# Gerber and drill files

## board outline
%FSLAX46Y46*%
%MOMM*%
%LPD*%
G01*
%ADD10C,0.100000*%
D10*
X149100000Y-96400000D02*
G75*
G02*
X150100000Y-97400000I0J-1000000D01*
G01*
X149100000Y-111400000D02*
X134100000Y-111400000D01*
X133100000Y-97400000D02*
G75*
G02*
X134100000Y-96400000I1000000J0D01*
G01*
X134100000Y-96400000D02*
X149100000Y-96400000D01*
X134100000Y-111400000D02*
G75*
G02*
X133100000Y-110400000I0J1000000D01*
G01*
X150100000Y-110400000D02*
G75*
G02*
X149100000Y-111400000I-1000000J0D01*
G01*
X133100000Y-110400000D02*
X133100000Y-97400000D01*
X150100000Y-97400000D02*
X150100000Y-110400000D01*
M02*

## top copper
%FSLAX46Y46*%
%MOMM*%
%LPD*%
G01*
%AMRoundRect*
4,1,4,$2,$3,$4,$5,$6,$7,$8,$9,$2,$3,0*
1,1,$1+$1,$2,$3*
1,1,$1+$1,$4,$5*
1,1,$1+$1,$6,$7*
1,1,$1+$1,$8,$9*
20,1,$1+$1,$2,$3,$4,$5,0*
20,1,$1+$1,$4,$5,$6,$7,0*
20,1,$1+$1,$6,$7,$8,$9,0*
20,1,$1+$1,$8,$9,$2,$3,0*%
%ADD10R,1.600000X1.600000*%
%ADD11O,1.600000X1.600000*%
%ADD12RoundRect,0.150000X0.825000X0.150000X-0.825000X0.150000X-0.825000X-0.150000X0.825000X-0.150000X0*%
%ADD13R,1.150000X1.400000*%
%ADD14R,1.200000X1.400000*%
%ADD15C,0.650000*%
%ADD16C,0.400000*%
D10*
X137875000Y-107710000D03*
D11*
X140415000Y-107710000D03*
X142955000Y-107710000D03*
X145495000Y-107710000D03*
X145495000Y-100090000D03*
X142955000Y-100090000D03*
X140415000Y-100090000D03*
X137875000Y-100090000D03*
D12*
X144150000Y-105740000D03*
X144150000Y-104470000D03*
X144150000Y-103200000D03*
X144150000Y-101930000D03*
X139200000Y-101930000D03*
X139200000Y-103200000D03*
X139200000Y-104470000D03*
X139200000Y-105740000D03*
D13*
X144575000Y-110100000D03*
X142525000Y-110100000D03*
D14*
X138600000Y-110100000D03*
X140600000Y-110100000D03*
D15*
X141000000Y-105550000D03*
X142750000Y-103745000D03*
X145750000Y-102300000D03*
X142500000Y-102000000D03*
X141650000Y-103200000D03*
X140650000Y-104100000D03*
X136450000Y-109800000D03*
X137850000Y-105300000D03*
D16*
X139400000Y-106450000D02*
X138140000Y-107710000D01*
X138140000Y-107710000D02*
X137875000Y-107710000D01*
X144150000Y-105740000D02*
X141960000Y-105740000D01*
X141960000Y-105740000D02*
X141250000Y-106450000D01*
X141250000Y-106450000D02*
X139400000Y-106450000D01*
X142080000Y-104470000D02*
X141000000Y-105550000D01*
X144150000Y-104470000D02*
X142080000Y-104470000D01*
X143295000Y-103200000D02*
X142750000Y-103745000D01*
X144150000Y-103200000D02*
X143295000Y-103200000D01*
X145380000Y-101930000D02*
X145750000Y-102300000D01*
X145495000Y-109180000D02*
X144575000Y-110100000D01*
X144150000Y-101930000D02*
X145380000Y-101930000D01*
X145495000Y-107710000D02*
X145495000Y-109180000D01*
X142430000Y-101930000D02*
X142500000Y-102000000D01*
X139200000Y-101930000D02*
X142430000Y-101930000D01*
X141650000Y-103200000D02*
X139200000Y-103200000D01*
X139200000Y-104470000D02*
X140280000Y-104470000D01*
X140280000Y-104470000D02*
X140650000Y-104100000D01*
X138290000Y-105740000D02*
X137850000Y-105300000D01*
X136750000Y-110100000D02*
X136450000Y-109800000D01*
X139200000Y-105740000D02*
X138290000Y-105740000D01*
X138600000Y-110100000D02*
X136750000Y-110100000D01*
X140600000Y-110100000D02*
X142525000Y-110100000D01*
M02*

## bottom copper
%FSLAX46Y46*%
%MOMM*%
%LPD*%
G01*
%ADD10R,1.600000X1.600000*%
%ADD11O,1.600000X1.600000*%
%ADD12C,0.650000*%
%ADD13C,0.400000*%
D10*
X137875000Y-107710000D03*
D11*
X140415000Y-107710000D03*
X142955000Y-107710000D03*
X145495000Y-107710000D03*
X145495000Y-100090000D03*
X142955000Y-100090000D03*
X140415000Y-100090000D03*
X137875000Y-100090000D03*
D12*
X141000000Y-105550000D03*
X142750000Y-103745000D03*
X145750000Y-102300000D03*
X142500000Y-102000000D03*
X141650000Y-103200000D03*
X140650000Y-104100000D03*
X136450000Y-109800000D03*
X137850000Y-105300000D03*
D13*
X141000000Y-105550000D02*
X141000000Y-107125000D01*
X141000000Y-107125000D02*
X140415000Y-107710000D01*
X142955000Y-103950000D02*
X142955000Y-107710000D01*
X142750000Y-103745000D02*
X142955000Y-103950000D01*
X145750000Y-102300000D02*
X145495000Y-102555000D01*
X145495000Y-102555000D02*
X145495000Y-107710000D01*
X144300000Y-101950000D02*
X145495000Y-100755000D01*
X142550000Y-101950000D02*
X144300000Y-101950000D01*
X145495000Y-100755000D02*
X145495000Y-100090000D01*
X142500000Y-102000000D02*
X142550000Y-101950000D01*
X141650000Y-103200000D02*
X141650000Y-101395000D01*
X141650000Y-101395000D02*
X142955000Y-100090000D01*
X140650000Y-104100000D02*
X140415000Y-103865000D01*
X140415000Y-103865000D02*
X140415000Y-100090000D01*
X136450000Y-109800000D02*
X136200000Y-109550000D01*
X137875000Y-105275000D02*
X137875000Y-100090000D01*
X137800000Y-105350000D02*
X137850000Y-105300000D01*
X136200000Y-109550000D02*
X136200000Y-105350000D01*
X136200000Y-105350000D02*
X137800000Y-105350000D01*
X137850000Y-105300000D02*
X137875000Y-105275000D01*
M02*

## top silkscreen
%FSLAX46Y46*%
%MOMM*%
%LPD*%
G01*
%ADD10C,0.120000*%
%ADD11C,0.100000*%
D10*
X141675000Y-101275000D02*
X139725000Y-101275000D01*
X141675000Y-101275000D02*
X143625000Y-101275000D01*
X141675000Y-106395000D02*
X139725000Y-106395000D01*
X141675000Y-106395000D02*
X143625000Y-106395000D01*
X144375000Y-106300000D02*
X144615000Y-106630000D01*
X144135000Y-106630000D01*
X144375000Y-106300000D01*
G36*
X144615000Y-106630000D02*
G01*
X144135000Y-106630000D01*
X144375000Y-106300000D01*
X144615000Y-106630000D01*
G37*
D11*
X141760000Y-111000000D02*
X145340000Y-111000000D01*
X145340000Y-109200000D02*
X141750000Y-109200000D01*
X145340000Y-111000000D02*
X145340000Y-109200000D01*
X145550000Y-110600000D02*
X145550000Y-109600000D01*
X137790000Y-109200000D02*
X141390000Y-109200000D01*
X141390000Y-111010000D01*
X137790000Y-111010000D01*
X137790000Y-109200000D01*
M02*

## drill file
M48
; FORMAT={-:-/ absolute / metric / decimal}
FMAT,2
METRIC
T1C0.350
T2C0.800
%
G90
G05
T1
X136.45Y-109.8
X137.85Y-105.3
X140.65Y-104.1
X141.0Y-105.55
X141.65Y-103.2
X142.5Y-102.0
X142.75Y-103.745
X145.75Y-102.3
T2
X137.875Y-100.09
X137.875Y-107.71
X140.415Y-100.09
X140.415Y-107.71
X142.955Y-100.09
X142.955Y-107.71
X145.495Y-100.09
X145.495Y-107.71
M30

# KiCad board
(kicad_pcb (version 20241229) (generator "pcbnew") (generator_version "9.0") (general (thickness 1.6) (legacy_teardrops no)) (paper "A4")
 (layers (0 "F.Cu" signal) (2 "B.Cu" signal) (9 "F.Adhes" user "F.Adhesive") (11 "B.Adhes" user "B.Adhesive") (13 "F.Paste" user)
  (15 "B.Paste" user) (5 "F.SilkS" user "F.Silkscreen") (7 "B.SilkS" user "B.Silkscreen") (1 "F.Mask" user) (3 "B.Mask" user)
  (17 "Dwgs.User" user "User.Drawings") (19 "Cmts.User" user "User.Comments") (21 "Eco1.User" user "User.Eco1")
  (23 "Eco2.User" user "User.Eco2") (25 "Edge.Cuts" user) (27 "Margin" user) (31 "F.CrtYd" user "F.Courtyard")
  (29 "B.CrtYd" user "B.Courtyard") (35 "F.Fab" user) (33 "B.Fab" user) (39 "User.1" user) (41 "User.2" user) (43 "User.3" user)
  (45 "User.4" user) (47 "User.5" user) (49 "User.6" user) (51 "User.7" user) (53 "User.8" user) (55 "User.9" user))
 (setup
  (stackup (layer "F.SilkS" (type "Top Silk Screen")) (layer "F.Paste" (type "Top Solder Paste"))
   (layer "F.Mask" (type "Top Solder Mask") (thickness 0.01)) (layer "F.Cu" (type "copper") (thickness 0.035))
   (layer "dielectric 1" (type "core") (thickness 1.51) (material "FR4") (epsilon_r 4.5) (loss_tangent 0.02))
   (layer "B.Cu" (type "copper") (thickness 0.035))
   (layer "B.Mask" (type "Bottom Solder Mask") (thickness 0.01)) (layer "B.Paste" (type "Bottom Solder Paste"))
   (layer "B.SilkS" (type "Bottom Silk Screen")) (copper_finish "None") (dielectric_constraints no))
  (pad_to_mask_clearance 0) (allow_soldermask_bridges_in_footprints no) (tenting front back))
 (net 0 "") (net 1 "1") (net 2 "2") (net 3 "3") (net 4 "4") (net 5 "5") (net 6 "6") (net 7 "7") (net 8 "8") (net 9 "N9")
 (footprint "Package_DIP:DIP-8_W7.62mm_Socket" (layer "F.Cu") (at 137.875 107.71 90)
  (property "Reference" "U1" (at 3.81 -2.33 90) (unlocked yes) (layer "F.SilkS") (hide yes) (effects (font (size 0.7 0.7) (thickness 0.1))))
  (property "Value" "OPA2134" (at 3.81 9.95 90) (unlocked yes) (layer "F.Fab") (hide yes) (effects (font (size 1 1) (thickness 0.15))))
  (pad "1" thru_hole rect (at 0 0 90) (size 1.6 1.6) (drill 0.8) (layers "*.Cu" "*.Mask") (remove_unused_layers no) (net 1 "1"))
  (pad "2" thru_hole oval (at 0 2.54 90) (size 1.6 1.6) (drill 0.8) (layers "*.Cu" "*.Mask") (remove_unused_layers no) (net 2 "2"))
  (pad "3" thru_hole oval (at 0 5.08 90) (size 1.6 1.6) (drill 0.8) (layers "*.Cu" "*.Mask") (remove_unused_layers no) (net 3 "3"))
  (pad "4" thru_hole oval (at 0 7.62 90) (size 1.6 1.6) (drill 0.8) (layers "*.Cu" "*.Mask") (remove_unused_layers no) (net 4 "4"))
  (pad "5" thru_hole oval (at 7.62 7.62 90) (size 1.6 1.6) (drill 0.8) (layers "*.Cu" "*.Mask") (remove_unused_layers no) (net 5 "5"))
  (pad "6" thru_hole oval (at 7.62 5.08 90) (size 1.6 1.6) (drill 0.8) (layers "*.Cu" "*.Mask") (remove_unused_layers no) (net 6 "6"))
  (pad "7" thru_hole oval (at 7.62 2.54 90) (size 1.6 1.6) (drill 0.8) (layers "*.Cu" "*.Mask") (remove_unused_layers no) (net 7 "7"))
  (pad "8" thru_hole oval (at 7.62 0 90) (size 1.6 1.6) (drill 0.8) (layers "*.Cu" "*.Mask") (remove_unused_layers no) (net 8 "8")))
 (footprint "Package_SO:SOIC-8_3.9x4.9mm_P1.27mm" (layer "F.Cu") (at 141.675 103.835 180)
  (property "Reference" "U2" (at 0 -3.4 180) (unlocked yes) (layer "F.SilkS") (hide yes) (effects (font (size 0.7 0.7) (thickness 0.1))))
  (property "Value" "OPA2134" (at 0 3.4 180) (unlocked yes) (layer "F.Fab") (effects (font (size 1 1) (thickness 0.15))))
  (fp_line (start 0 2.56) (end 1.95 2.56) (stroke (width 0.12) (type solid)) (layer "F.SilkS"))
  (fp_line (start 0 2.56) (end -1.95 2.56) (stroke (width 0.12) (type solid)) (layer "F.SilkS"))
  (fp_line (start 0 -2.56) (end 1.95 -2.56) (stroke (width 0.12) (type solid)) (layer "F.SilkS"))
  (fp_line (start 0 -2.56) (end -1.95 -2.56) (stroke (width 0.12) (type solid)) (layer "F.SilkS"))
  (fp_poly
   (pts (xy -2.7 -2.465) (xy -2.94 -2.795) (xy -2.46 -2.795) (xy -2.7 -2.465)) (stroke (width 0.12) (type solid)) (fill yes)
   (layer "F.SilkS"))
  (pad "1" smd roundrect (at -2.475 -1.905 180) (size 1.95 0.6) (layers "F.Cu" "F.Mask" "F.Paste") (roundrect_rratio 0.25) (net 1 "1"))
  (pad "2" smd roundrect (at -2.475 -0.635 180) (size 1.95 0.6) (layers "F.Cu" "F.Mask" "F.Paste") (roundrect_rratio 0.25) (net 2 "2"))
  (pad "3" smd roundrect (at -2.475 0.635 180) (size 1.95 0.6) (layers "F.Cu" "F.Mask" "F.Paste") (roundrect_rratio 0.25) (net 3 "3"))
  (pad "4" smd roundrect (at -2.475 1.905 180) (size 1.95 0.6) (layers "F.Cu" "F.Mask" "F.Paste") (roundrect_rratio 0.25) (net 4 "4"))
  (pad "5" smd roundrect (at 2.475 1.905 180) (size 1.95 0.6) (layers "F.Cu" "F.Mask" "F.Paste") (roundrect_rratio 0.25) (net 5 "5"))
  (pad "6" smd roundrect (at 2.475 0.635 180) (size 1.95 0.6) (layers "F.Cu" "F.Mask" "F.Paste") (roundrect_rratio 0.25) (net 6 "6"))
  (pad "7" smd roundrect (at 2.475 -0.635 180) (size 1.95 0.6) (layers "F.Cu" "F.Mask" "F.Paste") (roundrect_rratio 0.25) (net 7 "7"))
  (pad "8" smd roundrect (at 2.475 -1.905 180) (size 1.95 0.6) (layers "F.Cu" "F.Mask" "F.Paste") (roundrect_rratio 0.25) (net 8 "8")))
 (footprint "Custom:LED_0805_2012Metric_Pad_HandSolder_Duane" (layer "F.Cu") (at 143.55 110.1 180)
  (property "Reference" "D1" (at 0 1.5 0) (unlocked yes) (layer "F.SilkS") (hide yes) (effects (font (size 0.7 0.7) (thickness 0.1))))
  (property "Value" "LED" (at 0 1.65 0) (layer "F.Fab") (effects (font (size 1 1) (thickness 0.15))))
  (fp_line (start 1.79 -0.9) (end -1.79 -0.9) (stroke (width 0.1) (type default)) (layer "F.SilkS"))
  (fp_line (start -1.79 0.9) (end 1.8 0.9) (stroke (width 0.1) (type default)) (layer "F.SilkS"))
  (fp_line (start -1.79 -0.9) (end -1.79 0.9) (stroke (width 0.1) (type default)) (layer "F.SilkS"))
  (fp_line (start -2 -0.5) (end -2 0.5) (stroke (width 0.1) (type default)) (layer "F.SilkS"))
  (pad "1" smd rect (at -1.025 0 180) (size 1.15 1.4) (layers "F.Cu" "F.Mask" "F.Paste") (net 4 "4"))
  (pad "2" smd rect (at 1.025 0 180) (size 1.15 1.4) (layers "F.Cu" "F.Mask" "F.Paste") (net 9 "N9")))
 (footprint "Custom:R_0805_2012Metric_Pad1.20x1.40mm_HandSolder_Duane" (layer "F.Cu") (at 139.6 110.1)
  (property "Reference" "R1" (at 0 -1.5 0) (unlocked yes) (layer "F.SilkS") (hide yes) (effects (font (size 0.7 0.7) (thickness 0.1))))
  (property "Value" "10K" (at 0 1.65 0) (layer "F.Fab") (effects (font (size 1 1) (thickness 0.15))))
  (fp_rect (start -1.81 -0.9) (end 1.79 0.91) (stroke (width 0.1) (type default)) (fill no) (layer "F.SilkS"))
  (pad "1" smd rect (at -1 0) (size 1.2 1.4) (layers "F.Cu" "F.Mask" "F.Paste") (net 8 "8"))
  (pad "2" smd rect (at 1 0) (size 1.2 1.4) (layers "F.Cu" "F.Mask" "F.Paste") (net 9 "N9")))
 (gr_arc (start 149.1 96.4) (mid 149.807107 96.692893) (end 150.1 97.4) (stroke (width 0.1) (type default)) (layer "Edge.Cuts"))
 (gr_line (start 149.1 111.4) (end 134.1 111.4) (stroke (width 0.1) (type default)) (layer "Edge.Cuts"))
 (gr_arc (start 133.1 97.4) (mid 133.392893 96.692893) (end 134.1 96.4) (stroke (width 0.1) (type default)) (layer "Edge.Cuts"))
 (gr_line (start 134.1 96.4) (end 149.1 96.4) (stroke (width 0.1) (type default)) (layer "Edge.Cuts"))
 (gr_arc (start 134.1 111.4) (mid 133.392893 111.107107) (end 133.1 110.4) (stroke (width 0.1) (type default)) (layer "Edge.Cuts"))
 (gr_arc (start 150.1 110.4) (mid 149.807107 111.107107) (end 149.1 111.4) (stroke (width 0.1) (type default)) (layer "Edge.Cuts"))
 (gr_line (start 133.1 110.4) (end 133.1 97.4) (stroke (width 0.1) (type default)) (layer "Edge.Cuts"))
 (gr_line (start 150.1 97.4) (end 150.1 110.4) (stroke (width 0.1) (type default)) (layer "Edge.Cuts"))
 (segment (start 139.4 106.45) (end 138.14 107.71) (width 0.4) (layer "F.Cu") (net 1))
 (segment (start 138.14 107.71) (end 137.875 107.71) (width 0.4) (layer "F.Cu") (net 1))
 (segment (start 144.15 105.74) (end 141.96 105.74) (width 0.4) (layer "F.Cu") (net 1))
 (segment (start 141.96 105.74) (end 141.25 106.45) (width 0.4) (layer "F.Cu") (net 1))
 (segment (start 141.25 106.45) (end 139.4 106.45) (width 0.4) (layer "F.Cu") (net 1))
 (segment (start 142.08 104.47) (end 141 105.55) (width 0.4) (layer "F.Cu") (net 2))
 (segment (start 144.15 104.47) (end 142.08 104.47) (width 0.4) (layer "F.Cu") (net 2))
 (via (at 141 105.55) (size 0.65) (drill 0.35) (layers "F.Cu" "B.Cu") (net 2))
 (segment (start 141 105.55) (end 141 107.125) (width 0.4) (layer "B.Cu") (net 2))
 (segment (start 141 107.125) (end 140.415 107.71) (width 0.4) (layer "B.Cu") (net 2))
 (segment (start 143.295 103.2) (end 142.75 103.745) (width 0.4) (layer "F.Cu") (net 3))
 (segment (start 144.15 103.2) (end 143.295 103.2) (width 0.4) (layer "F.Cu") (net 3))
 (via (at 142.75 103.745) (size 0.65) (drill 0.35) (layers "F.Cu" "B.Cu") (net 3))
 (segment (start 142.955 103.95) (end 142.955 107.71) (width 0.4) (layer "B.Cu") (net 3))
 (segment (start 142.75 103.745) (end 142.955 103.95) (width 0.4) (layer "B.Cu") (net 3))
 (segment (start 145.38 101.93) (end 145.75 102.3) (width 0.4) (layer "F.Cu") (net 4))
 (segment (start 145.495 109.18) (end 144.575 110.1) (width 0.4) (layer "F.Cu") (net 4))
 (segment (start 144.15 101.93) (end 145.38 101.93) (width 0.4) (layer "F.Cu") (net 4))
 (segment (start 145.495 107.71) (end 145.495 109.18) (width 0.4) (layer "F.Cu") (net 4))
 (via (at 145.75 102.3) (size 0.65) (drill 0.35) (layers "F.Cu" "B.Cu") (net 4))
 (segment (start 145.75 102.3) (end 145.495 102.555) (width 0.4) (layer "B.Cu") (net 4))
 (segment (start 145.495 102.555) (end 145.495 107.71) (width 0.4) (layer "B.Cu") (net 4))
 (segment (start 142.43 101.93) (end 142.5 102) (width 0.4) (layer "F.Cu") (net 5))
 (segment (start 139.2 101.93) (end 142.43 101.93) (width 0.4) (layer "F.Cu") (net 5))
 (via (at 142.5 102) (size 0.65) (drill 0.35) (layers "F.Cu" "B.Cu") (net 5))
 (segment (start 144.3 101.95) (end 145.495 100.755) (width 0.4) (layer "B.Cu") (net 5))
 (segment (start 142.55 101.95) (end 144.3 101.95) (width 0.4) (layer "B.Cu") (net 5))
 (segment (start 145.495 100.755) (end 145.495 100.09) (width 0.4) (layer "B.Cu") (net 5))
 (segment (start 142.5 102) (end 142.55 101.95) (width 0.4) (layer "B.Cu") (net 5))
 (segment (start 141.65 103.2) (end 139.2 103.2) (width 0.4) (layer "F.Cu") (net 6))
 (via (at 141.65 103.2) (size 0.65) (drill 0.35) (layers "F.Cu" "B.Cu") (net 6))
 (segment (start 141.65 103.2) (end 141.65 101.395) (width 0.4) (layer "B.Cu") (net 6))
 (segment (start 141.65 101.395) (end 142.955 100.09) (width 0.4) (layer "B.Cu") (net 6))
 (segment (start 139.2 104.47) (end 140.28 104.47) (width 0.4) (layer "F.Cu") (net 7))
 (segment (start 140.28 104.47) (end 140.65 104.1) (width 0.4) (layer "F.Cu") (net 7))
 (via (at 140.65 104.1) (size 0.65) (drill 0.35) (layers "F.Cu" "B.Cu") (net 7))
 (segment (start 140.65 104.1) (end 140.415 103.865) (width 0.4) (layer "B.Cu") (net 7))
 (segment (start 140.415 103.865) (end 140.415 100.09) (width 0.4) (layer "B.Cu") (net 7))
 (segment (start 138.29 105.74) (end 137.85 105.3) (width 0.4) (layer "F.Cu") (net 8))
 (segment (start 136.75 110.1) (end 136.45 109.8) (width 0.4) (layer "F.Cu") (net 8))
 (segment (start 139.2 105.74) (end 138.29 105.74) (width 0.4) (layer "F.Cu") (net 8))
 (segment (start 138.6 110.1) (end 136.75 110.1) (width 0.4) (layer "F.Cu") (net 8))
 (via (at 136.45 109.8) (size 0.65) (drill 0.35) (layers "F.Cu" "B.Cu") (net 8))
 (via (at 137.85 105.3) (size 0.65) (drill 0.35) (layers "F.Cu" "B.Cu") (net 8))
 (segment (start 136.45 109.8) (end 136.2 109.55) (width 0.4) (layer "B.Cu") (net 8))
 (segment (start 137.875 105.275) (end 137.875 100.09) (width 0.4) (layer "B.Cu") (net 8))
 (segment (start 137.8 105.35) (end 137.85 105.3) (width 0.4) (layer "B.Cu") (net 8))
 (segment (start 136.2 109.55) (end 136.2 105.35) (width 0.4) (layer "B.Cu") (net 8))
 (segment (start 136.2 105.35) (end 137.8 105.35) (width 0.4) (layer "B.Cu") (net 8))
 (segment (start 137.85 105.3) (end 137.875 105.275) (width 0.4) (layer "B.Cu") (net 8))
 (segment (start 140.6 110.1) (end 142.525 110.1) (width 0.4) (layer "F.Cu") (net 9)))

